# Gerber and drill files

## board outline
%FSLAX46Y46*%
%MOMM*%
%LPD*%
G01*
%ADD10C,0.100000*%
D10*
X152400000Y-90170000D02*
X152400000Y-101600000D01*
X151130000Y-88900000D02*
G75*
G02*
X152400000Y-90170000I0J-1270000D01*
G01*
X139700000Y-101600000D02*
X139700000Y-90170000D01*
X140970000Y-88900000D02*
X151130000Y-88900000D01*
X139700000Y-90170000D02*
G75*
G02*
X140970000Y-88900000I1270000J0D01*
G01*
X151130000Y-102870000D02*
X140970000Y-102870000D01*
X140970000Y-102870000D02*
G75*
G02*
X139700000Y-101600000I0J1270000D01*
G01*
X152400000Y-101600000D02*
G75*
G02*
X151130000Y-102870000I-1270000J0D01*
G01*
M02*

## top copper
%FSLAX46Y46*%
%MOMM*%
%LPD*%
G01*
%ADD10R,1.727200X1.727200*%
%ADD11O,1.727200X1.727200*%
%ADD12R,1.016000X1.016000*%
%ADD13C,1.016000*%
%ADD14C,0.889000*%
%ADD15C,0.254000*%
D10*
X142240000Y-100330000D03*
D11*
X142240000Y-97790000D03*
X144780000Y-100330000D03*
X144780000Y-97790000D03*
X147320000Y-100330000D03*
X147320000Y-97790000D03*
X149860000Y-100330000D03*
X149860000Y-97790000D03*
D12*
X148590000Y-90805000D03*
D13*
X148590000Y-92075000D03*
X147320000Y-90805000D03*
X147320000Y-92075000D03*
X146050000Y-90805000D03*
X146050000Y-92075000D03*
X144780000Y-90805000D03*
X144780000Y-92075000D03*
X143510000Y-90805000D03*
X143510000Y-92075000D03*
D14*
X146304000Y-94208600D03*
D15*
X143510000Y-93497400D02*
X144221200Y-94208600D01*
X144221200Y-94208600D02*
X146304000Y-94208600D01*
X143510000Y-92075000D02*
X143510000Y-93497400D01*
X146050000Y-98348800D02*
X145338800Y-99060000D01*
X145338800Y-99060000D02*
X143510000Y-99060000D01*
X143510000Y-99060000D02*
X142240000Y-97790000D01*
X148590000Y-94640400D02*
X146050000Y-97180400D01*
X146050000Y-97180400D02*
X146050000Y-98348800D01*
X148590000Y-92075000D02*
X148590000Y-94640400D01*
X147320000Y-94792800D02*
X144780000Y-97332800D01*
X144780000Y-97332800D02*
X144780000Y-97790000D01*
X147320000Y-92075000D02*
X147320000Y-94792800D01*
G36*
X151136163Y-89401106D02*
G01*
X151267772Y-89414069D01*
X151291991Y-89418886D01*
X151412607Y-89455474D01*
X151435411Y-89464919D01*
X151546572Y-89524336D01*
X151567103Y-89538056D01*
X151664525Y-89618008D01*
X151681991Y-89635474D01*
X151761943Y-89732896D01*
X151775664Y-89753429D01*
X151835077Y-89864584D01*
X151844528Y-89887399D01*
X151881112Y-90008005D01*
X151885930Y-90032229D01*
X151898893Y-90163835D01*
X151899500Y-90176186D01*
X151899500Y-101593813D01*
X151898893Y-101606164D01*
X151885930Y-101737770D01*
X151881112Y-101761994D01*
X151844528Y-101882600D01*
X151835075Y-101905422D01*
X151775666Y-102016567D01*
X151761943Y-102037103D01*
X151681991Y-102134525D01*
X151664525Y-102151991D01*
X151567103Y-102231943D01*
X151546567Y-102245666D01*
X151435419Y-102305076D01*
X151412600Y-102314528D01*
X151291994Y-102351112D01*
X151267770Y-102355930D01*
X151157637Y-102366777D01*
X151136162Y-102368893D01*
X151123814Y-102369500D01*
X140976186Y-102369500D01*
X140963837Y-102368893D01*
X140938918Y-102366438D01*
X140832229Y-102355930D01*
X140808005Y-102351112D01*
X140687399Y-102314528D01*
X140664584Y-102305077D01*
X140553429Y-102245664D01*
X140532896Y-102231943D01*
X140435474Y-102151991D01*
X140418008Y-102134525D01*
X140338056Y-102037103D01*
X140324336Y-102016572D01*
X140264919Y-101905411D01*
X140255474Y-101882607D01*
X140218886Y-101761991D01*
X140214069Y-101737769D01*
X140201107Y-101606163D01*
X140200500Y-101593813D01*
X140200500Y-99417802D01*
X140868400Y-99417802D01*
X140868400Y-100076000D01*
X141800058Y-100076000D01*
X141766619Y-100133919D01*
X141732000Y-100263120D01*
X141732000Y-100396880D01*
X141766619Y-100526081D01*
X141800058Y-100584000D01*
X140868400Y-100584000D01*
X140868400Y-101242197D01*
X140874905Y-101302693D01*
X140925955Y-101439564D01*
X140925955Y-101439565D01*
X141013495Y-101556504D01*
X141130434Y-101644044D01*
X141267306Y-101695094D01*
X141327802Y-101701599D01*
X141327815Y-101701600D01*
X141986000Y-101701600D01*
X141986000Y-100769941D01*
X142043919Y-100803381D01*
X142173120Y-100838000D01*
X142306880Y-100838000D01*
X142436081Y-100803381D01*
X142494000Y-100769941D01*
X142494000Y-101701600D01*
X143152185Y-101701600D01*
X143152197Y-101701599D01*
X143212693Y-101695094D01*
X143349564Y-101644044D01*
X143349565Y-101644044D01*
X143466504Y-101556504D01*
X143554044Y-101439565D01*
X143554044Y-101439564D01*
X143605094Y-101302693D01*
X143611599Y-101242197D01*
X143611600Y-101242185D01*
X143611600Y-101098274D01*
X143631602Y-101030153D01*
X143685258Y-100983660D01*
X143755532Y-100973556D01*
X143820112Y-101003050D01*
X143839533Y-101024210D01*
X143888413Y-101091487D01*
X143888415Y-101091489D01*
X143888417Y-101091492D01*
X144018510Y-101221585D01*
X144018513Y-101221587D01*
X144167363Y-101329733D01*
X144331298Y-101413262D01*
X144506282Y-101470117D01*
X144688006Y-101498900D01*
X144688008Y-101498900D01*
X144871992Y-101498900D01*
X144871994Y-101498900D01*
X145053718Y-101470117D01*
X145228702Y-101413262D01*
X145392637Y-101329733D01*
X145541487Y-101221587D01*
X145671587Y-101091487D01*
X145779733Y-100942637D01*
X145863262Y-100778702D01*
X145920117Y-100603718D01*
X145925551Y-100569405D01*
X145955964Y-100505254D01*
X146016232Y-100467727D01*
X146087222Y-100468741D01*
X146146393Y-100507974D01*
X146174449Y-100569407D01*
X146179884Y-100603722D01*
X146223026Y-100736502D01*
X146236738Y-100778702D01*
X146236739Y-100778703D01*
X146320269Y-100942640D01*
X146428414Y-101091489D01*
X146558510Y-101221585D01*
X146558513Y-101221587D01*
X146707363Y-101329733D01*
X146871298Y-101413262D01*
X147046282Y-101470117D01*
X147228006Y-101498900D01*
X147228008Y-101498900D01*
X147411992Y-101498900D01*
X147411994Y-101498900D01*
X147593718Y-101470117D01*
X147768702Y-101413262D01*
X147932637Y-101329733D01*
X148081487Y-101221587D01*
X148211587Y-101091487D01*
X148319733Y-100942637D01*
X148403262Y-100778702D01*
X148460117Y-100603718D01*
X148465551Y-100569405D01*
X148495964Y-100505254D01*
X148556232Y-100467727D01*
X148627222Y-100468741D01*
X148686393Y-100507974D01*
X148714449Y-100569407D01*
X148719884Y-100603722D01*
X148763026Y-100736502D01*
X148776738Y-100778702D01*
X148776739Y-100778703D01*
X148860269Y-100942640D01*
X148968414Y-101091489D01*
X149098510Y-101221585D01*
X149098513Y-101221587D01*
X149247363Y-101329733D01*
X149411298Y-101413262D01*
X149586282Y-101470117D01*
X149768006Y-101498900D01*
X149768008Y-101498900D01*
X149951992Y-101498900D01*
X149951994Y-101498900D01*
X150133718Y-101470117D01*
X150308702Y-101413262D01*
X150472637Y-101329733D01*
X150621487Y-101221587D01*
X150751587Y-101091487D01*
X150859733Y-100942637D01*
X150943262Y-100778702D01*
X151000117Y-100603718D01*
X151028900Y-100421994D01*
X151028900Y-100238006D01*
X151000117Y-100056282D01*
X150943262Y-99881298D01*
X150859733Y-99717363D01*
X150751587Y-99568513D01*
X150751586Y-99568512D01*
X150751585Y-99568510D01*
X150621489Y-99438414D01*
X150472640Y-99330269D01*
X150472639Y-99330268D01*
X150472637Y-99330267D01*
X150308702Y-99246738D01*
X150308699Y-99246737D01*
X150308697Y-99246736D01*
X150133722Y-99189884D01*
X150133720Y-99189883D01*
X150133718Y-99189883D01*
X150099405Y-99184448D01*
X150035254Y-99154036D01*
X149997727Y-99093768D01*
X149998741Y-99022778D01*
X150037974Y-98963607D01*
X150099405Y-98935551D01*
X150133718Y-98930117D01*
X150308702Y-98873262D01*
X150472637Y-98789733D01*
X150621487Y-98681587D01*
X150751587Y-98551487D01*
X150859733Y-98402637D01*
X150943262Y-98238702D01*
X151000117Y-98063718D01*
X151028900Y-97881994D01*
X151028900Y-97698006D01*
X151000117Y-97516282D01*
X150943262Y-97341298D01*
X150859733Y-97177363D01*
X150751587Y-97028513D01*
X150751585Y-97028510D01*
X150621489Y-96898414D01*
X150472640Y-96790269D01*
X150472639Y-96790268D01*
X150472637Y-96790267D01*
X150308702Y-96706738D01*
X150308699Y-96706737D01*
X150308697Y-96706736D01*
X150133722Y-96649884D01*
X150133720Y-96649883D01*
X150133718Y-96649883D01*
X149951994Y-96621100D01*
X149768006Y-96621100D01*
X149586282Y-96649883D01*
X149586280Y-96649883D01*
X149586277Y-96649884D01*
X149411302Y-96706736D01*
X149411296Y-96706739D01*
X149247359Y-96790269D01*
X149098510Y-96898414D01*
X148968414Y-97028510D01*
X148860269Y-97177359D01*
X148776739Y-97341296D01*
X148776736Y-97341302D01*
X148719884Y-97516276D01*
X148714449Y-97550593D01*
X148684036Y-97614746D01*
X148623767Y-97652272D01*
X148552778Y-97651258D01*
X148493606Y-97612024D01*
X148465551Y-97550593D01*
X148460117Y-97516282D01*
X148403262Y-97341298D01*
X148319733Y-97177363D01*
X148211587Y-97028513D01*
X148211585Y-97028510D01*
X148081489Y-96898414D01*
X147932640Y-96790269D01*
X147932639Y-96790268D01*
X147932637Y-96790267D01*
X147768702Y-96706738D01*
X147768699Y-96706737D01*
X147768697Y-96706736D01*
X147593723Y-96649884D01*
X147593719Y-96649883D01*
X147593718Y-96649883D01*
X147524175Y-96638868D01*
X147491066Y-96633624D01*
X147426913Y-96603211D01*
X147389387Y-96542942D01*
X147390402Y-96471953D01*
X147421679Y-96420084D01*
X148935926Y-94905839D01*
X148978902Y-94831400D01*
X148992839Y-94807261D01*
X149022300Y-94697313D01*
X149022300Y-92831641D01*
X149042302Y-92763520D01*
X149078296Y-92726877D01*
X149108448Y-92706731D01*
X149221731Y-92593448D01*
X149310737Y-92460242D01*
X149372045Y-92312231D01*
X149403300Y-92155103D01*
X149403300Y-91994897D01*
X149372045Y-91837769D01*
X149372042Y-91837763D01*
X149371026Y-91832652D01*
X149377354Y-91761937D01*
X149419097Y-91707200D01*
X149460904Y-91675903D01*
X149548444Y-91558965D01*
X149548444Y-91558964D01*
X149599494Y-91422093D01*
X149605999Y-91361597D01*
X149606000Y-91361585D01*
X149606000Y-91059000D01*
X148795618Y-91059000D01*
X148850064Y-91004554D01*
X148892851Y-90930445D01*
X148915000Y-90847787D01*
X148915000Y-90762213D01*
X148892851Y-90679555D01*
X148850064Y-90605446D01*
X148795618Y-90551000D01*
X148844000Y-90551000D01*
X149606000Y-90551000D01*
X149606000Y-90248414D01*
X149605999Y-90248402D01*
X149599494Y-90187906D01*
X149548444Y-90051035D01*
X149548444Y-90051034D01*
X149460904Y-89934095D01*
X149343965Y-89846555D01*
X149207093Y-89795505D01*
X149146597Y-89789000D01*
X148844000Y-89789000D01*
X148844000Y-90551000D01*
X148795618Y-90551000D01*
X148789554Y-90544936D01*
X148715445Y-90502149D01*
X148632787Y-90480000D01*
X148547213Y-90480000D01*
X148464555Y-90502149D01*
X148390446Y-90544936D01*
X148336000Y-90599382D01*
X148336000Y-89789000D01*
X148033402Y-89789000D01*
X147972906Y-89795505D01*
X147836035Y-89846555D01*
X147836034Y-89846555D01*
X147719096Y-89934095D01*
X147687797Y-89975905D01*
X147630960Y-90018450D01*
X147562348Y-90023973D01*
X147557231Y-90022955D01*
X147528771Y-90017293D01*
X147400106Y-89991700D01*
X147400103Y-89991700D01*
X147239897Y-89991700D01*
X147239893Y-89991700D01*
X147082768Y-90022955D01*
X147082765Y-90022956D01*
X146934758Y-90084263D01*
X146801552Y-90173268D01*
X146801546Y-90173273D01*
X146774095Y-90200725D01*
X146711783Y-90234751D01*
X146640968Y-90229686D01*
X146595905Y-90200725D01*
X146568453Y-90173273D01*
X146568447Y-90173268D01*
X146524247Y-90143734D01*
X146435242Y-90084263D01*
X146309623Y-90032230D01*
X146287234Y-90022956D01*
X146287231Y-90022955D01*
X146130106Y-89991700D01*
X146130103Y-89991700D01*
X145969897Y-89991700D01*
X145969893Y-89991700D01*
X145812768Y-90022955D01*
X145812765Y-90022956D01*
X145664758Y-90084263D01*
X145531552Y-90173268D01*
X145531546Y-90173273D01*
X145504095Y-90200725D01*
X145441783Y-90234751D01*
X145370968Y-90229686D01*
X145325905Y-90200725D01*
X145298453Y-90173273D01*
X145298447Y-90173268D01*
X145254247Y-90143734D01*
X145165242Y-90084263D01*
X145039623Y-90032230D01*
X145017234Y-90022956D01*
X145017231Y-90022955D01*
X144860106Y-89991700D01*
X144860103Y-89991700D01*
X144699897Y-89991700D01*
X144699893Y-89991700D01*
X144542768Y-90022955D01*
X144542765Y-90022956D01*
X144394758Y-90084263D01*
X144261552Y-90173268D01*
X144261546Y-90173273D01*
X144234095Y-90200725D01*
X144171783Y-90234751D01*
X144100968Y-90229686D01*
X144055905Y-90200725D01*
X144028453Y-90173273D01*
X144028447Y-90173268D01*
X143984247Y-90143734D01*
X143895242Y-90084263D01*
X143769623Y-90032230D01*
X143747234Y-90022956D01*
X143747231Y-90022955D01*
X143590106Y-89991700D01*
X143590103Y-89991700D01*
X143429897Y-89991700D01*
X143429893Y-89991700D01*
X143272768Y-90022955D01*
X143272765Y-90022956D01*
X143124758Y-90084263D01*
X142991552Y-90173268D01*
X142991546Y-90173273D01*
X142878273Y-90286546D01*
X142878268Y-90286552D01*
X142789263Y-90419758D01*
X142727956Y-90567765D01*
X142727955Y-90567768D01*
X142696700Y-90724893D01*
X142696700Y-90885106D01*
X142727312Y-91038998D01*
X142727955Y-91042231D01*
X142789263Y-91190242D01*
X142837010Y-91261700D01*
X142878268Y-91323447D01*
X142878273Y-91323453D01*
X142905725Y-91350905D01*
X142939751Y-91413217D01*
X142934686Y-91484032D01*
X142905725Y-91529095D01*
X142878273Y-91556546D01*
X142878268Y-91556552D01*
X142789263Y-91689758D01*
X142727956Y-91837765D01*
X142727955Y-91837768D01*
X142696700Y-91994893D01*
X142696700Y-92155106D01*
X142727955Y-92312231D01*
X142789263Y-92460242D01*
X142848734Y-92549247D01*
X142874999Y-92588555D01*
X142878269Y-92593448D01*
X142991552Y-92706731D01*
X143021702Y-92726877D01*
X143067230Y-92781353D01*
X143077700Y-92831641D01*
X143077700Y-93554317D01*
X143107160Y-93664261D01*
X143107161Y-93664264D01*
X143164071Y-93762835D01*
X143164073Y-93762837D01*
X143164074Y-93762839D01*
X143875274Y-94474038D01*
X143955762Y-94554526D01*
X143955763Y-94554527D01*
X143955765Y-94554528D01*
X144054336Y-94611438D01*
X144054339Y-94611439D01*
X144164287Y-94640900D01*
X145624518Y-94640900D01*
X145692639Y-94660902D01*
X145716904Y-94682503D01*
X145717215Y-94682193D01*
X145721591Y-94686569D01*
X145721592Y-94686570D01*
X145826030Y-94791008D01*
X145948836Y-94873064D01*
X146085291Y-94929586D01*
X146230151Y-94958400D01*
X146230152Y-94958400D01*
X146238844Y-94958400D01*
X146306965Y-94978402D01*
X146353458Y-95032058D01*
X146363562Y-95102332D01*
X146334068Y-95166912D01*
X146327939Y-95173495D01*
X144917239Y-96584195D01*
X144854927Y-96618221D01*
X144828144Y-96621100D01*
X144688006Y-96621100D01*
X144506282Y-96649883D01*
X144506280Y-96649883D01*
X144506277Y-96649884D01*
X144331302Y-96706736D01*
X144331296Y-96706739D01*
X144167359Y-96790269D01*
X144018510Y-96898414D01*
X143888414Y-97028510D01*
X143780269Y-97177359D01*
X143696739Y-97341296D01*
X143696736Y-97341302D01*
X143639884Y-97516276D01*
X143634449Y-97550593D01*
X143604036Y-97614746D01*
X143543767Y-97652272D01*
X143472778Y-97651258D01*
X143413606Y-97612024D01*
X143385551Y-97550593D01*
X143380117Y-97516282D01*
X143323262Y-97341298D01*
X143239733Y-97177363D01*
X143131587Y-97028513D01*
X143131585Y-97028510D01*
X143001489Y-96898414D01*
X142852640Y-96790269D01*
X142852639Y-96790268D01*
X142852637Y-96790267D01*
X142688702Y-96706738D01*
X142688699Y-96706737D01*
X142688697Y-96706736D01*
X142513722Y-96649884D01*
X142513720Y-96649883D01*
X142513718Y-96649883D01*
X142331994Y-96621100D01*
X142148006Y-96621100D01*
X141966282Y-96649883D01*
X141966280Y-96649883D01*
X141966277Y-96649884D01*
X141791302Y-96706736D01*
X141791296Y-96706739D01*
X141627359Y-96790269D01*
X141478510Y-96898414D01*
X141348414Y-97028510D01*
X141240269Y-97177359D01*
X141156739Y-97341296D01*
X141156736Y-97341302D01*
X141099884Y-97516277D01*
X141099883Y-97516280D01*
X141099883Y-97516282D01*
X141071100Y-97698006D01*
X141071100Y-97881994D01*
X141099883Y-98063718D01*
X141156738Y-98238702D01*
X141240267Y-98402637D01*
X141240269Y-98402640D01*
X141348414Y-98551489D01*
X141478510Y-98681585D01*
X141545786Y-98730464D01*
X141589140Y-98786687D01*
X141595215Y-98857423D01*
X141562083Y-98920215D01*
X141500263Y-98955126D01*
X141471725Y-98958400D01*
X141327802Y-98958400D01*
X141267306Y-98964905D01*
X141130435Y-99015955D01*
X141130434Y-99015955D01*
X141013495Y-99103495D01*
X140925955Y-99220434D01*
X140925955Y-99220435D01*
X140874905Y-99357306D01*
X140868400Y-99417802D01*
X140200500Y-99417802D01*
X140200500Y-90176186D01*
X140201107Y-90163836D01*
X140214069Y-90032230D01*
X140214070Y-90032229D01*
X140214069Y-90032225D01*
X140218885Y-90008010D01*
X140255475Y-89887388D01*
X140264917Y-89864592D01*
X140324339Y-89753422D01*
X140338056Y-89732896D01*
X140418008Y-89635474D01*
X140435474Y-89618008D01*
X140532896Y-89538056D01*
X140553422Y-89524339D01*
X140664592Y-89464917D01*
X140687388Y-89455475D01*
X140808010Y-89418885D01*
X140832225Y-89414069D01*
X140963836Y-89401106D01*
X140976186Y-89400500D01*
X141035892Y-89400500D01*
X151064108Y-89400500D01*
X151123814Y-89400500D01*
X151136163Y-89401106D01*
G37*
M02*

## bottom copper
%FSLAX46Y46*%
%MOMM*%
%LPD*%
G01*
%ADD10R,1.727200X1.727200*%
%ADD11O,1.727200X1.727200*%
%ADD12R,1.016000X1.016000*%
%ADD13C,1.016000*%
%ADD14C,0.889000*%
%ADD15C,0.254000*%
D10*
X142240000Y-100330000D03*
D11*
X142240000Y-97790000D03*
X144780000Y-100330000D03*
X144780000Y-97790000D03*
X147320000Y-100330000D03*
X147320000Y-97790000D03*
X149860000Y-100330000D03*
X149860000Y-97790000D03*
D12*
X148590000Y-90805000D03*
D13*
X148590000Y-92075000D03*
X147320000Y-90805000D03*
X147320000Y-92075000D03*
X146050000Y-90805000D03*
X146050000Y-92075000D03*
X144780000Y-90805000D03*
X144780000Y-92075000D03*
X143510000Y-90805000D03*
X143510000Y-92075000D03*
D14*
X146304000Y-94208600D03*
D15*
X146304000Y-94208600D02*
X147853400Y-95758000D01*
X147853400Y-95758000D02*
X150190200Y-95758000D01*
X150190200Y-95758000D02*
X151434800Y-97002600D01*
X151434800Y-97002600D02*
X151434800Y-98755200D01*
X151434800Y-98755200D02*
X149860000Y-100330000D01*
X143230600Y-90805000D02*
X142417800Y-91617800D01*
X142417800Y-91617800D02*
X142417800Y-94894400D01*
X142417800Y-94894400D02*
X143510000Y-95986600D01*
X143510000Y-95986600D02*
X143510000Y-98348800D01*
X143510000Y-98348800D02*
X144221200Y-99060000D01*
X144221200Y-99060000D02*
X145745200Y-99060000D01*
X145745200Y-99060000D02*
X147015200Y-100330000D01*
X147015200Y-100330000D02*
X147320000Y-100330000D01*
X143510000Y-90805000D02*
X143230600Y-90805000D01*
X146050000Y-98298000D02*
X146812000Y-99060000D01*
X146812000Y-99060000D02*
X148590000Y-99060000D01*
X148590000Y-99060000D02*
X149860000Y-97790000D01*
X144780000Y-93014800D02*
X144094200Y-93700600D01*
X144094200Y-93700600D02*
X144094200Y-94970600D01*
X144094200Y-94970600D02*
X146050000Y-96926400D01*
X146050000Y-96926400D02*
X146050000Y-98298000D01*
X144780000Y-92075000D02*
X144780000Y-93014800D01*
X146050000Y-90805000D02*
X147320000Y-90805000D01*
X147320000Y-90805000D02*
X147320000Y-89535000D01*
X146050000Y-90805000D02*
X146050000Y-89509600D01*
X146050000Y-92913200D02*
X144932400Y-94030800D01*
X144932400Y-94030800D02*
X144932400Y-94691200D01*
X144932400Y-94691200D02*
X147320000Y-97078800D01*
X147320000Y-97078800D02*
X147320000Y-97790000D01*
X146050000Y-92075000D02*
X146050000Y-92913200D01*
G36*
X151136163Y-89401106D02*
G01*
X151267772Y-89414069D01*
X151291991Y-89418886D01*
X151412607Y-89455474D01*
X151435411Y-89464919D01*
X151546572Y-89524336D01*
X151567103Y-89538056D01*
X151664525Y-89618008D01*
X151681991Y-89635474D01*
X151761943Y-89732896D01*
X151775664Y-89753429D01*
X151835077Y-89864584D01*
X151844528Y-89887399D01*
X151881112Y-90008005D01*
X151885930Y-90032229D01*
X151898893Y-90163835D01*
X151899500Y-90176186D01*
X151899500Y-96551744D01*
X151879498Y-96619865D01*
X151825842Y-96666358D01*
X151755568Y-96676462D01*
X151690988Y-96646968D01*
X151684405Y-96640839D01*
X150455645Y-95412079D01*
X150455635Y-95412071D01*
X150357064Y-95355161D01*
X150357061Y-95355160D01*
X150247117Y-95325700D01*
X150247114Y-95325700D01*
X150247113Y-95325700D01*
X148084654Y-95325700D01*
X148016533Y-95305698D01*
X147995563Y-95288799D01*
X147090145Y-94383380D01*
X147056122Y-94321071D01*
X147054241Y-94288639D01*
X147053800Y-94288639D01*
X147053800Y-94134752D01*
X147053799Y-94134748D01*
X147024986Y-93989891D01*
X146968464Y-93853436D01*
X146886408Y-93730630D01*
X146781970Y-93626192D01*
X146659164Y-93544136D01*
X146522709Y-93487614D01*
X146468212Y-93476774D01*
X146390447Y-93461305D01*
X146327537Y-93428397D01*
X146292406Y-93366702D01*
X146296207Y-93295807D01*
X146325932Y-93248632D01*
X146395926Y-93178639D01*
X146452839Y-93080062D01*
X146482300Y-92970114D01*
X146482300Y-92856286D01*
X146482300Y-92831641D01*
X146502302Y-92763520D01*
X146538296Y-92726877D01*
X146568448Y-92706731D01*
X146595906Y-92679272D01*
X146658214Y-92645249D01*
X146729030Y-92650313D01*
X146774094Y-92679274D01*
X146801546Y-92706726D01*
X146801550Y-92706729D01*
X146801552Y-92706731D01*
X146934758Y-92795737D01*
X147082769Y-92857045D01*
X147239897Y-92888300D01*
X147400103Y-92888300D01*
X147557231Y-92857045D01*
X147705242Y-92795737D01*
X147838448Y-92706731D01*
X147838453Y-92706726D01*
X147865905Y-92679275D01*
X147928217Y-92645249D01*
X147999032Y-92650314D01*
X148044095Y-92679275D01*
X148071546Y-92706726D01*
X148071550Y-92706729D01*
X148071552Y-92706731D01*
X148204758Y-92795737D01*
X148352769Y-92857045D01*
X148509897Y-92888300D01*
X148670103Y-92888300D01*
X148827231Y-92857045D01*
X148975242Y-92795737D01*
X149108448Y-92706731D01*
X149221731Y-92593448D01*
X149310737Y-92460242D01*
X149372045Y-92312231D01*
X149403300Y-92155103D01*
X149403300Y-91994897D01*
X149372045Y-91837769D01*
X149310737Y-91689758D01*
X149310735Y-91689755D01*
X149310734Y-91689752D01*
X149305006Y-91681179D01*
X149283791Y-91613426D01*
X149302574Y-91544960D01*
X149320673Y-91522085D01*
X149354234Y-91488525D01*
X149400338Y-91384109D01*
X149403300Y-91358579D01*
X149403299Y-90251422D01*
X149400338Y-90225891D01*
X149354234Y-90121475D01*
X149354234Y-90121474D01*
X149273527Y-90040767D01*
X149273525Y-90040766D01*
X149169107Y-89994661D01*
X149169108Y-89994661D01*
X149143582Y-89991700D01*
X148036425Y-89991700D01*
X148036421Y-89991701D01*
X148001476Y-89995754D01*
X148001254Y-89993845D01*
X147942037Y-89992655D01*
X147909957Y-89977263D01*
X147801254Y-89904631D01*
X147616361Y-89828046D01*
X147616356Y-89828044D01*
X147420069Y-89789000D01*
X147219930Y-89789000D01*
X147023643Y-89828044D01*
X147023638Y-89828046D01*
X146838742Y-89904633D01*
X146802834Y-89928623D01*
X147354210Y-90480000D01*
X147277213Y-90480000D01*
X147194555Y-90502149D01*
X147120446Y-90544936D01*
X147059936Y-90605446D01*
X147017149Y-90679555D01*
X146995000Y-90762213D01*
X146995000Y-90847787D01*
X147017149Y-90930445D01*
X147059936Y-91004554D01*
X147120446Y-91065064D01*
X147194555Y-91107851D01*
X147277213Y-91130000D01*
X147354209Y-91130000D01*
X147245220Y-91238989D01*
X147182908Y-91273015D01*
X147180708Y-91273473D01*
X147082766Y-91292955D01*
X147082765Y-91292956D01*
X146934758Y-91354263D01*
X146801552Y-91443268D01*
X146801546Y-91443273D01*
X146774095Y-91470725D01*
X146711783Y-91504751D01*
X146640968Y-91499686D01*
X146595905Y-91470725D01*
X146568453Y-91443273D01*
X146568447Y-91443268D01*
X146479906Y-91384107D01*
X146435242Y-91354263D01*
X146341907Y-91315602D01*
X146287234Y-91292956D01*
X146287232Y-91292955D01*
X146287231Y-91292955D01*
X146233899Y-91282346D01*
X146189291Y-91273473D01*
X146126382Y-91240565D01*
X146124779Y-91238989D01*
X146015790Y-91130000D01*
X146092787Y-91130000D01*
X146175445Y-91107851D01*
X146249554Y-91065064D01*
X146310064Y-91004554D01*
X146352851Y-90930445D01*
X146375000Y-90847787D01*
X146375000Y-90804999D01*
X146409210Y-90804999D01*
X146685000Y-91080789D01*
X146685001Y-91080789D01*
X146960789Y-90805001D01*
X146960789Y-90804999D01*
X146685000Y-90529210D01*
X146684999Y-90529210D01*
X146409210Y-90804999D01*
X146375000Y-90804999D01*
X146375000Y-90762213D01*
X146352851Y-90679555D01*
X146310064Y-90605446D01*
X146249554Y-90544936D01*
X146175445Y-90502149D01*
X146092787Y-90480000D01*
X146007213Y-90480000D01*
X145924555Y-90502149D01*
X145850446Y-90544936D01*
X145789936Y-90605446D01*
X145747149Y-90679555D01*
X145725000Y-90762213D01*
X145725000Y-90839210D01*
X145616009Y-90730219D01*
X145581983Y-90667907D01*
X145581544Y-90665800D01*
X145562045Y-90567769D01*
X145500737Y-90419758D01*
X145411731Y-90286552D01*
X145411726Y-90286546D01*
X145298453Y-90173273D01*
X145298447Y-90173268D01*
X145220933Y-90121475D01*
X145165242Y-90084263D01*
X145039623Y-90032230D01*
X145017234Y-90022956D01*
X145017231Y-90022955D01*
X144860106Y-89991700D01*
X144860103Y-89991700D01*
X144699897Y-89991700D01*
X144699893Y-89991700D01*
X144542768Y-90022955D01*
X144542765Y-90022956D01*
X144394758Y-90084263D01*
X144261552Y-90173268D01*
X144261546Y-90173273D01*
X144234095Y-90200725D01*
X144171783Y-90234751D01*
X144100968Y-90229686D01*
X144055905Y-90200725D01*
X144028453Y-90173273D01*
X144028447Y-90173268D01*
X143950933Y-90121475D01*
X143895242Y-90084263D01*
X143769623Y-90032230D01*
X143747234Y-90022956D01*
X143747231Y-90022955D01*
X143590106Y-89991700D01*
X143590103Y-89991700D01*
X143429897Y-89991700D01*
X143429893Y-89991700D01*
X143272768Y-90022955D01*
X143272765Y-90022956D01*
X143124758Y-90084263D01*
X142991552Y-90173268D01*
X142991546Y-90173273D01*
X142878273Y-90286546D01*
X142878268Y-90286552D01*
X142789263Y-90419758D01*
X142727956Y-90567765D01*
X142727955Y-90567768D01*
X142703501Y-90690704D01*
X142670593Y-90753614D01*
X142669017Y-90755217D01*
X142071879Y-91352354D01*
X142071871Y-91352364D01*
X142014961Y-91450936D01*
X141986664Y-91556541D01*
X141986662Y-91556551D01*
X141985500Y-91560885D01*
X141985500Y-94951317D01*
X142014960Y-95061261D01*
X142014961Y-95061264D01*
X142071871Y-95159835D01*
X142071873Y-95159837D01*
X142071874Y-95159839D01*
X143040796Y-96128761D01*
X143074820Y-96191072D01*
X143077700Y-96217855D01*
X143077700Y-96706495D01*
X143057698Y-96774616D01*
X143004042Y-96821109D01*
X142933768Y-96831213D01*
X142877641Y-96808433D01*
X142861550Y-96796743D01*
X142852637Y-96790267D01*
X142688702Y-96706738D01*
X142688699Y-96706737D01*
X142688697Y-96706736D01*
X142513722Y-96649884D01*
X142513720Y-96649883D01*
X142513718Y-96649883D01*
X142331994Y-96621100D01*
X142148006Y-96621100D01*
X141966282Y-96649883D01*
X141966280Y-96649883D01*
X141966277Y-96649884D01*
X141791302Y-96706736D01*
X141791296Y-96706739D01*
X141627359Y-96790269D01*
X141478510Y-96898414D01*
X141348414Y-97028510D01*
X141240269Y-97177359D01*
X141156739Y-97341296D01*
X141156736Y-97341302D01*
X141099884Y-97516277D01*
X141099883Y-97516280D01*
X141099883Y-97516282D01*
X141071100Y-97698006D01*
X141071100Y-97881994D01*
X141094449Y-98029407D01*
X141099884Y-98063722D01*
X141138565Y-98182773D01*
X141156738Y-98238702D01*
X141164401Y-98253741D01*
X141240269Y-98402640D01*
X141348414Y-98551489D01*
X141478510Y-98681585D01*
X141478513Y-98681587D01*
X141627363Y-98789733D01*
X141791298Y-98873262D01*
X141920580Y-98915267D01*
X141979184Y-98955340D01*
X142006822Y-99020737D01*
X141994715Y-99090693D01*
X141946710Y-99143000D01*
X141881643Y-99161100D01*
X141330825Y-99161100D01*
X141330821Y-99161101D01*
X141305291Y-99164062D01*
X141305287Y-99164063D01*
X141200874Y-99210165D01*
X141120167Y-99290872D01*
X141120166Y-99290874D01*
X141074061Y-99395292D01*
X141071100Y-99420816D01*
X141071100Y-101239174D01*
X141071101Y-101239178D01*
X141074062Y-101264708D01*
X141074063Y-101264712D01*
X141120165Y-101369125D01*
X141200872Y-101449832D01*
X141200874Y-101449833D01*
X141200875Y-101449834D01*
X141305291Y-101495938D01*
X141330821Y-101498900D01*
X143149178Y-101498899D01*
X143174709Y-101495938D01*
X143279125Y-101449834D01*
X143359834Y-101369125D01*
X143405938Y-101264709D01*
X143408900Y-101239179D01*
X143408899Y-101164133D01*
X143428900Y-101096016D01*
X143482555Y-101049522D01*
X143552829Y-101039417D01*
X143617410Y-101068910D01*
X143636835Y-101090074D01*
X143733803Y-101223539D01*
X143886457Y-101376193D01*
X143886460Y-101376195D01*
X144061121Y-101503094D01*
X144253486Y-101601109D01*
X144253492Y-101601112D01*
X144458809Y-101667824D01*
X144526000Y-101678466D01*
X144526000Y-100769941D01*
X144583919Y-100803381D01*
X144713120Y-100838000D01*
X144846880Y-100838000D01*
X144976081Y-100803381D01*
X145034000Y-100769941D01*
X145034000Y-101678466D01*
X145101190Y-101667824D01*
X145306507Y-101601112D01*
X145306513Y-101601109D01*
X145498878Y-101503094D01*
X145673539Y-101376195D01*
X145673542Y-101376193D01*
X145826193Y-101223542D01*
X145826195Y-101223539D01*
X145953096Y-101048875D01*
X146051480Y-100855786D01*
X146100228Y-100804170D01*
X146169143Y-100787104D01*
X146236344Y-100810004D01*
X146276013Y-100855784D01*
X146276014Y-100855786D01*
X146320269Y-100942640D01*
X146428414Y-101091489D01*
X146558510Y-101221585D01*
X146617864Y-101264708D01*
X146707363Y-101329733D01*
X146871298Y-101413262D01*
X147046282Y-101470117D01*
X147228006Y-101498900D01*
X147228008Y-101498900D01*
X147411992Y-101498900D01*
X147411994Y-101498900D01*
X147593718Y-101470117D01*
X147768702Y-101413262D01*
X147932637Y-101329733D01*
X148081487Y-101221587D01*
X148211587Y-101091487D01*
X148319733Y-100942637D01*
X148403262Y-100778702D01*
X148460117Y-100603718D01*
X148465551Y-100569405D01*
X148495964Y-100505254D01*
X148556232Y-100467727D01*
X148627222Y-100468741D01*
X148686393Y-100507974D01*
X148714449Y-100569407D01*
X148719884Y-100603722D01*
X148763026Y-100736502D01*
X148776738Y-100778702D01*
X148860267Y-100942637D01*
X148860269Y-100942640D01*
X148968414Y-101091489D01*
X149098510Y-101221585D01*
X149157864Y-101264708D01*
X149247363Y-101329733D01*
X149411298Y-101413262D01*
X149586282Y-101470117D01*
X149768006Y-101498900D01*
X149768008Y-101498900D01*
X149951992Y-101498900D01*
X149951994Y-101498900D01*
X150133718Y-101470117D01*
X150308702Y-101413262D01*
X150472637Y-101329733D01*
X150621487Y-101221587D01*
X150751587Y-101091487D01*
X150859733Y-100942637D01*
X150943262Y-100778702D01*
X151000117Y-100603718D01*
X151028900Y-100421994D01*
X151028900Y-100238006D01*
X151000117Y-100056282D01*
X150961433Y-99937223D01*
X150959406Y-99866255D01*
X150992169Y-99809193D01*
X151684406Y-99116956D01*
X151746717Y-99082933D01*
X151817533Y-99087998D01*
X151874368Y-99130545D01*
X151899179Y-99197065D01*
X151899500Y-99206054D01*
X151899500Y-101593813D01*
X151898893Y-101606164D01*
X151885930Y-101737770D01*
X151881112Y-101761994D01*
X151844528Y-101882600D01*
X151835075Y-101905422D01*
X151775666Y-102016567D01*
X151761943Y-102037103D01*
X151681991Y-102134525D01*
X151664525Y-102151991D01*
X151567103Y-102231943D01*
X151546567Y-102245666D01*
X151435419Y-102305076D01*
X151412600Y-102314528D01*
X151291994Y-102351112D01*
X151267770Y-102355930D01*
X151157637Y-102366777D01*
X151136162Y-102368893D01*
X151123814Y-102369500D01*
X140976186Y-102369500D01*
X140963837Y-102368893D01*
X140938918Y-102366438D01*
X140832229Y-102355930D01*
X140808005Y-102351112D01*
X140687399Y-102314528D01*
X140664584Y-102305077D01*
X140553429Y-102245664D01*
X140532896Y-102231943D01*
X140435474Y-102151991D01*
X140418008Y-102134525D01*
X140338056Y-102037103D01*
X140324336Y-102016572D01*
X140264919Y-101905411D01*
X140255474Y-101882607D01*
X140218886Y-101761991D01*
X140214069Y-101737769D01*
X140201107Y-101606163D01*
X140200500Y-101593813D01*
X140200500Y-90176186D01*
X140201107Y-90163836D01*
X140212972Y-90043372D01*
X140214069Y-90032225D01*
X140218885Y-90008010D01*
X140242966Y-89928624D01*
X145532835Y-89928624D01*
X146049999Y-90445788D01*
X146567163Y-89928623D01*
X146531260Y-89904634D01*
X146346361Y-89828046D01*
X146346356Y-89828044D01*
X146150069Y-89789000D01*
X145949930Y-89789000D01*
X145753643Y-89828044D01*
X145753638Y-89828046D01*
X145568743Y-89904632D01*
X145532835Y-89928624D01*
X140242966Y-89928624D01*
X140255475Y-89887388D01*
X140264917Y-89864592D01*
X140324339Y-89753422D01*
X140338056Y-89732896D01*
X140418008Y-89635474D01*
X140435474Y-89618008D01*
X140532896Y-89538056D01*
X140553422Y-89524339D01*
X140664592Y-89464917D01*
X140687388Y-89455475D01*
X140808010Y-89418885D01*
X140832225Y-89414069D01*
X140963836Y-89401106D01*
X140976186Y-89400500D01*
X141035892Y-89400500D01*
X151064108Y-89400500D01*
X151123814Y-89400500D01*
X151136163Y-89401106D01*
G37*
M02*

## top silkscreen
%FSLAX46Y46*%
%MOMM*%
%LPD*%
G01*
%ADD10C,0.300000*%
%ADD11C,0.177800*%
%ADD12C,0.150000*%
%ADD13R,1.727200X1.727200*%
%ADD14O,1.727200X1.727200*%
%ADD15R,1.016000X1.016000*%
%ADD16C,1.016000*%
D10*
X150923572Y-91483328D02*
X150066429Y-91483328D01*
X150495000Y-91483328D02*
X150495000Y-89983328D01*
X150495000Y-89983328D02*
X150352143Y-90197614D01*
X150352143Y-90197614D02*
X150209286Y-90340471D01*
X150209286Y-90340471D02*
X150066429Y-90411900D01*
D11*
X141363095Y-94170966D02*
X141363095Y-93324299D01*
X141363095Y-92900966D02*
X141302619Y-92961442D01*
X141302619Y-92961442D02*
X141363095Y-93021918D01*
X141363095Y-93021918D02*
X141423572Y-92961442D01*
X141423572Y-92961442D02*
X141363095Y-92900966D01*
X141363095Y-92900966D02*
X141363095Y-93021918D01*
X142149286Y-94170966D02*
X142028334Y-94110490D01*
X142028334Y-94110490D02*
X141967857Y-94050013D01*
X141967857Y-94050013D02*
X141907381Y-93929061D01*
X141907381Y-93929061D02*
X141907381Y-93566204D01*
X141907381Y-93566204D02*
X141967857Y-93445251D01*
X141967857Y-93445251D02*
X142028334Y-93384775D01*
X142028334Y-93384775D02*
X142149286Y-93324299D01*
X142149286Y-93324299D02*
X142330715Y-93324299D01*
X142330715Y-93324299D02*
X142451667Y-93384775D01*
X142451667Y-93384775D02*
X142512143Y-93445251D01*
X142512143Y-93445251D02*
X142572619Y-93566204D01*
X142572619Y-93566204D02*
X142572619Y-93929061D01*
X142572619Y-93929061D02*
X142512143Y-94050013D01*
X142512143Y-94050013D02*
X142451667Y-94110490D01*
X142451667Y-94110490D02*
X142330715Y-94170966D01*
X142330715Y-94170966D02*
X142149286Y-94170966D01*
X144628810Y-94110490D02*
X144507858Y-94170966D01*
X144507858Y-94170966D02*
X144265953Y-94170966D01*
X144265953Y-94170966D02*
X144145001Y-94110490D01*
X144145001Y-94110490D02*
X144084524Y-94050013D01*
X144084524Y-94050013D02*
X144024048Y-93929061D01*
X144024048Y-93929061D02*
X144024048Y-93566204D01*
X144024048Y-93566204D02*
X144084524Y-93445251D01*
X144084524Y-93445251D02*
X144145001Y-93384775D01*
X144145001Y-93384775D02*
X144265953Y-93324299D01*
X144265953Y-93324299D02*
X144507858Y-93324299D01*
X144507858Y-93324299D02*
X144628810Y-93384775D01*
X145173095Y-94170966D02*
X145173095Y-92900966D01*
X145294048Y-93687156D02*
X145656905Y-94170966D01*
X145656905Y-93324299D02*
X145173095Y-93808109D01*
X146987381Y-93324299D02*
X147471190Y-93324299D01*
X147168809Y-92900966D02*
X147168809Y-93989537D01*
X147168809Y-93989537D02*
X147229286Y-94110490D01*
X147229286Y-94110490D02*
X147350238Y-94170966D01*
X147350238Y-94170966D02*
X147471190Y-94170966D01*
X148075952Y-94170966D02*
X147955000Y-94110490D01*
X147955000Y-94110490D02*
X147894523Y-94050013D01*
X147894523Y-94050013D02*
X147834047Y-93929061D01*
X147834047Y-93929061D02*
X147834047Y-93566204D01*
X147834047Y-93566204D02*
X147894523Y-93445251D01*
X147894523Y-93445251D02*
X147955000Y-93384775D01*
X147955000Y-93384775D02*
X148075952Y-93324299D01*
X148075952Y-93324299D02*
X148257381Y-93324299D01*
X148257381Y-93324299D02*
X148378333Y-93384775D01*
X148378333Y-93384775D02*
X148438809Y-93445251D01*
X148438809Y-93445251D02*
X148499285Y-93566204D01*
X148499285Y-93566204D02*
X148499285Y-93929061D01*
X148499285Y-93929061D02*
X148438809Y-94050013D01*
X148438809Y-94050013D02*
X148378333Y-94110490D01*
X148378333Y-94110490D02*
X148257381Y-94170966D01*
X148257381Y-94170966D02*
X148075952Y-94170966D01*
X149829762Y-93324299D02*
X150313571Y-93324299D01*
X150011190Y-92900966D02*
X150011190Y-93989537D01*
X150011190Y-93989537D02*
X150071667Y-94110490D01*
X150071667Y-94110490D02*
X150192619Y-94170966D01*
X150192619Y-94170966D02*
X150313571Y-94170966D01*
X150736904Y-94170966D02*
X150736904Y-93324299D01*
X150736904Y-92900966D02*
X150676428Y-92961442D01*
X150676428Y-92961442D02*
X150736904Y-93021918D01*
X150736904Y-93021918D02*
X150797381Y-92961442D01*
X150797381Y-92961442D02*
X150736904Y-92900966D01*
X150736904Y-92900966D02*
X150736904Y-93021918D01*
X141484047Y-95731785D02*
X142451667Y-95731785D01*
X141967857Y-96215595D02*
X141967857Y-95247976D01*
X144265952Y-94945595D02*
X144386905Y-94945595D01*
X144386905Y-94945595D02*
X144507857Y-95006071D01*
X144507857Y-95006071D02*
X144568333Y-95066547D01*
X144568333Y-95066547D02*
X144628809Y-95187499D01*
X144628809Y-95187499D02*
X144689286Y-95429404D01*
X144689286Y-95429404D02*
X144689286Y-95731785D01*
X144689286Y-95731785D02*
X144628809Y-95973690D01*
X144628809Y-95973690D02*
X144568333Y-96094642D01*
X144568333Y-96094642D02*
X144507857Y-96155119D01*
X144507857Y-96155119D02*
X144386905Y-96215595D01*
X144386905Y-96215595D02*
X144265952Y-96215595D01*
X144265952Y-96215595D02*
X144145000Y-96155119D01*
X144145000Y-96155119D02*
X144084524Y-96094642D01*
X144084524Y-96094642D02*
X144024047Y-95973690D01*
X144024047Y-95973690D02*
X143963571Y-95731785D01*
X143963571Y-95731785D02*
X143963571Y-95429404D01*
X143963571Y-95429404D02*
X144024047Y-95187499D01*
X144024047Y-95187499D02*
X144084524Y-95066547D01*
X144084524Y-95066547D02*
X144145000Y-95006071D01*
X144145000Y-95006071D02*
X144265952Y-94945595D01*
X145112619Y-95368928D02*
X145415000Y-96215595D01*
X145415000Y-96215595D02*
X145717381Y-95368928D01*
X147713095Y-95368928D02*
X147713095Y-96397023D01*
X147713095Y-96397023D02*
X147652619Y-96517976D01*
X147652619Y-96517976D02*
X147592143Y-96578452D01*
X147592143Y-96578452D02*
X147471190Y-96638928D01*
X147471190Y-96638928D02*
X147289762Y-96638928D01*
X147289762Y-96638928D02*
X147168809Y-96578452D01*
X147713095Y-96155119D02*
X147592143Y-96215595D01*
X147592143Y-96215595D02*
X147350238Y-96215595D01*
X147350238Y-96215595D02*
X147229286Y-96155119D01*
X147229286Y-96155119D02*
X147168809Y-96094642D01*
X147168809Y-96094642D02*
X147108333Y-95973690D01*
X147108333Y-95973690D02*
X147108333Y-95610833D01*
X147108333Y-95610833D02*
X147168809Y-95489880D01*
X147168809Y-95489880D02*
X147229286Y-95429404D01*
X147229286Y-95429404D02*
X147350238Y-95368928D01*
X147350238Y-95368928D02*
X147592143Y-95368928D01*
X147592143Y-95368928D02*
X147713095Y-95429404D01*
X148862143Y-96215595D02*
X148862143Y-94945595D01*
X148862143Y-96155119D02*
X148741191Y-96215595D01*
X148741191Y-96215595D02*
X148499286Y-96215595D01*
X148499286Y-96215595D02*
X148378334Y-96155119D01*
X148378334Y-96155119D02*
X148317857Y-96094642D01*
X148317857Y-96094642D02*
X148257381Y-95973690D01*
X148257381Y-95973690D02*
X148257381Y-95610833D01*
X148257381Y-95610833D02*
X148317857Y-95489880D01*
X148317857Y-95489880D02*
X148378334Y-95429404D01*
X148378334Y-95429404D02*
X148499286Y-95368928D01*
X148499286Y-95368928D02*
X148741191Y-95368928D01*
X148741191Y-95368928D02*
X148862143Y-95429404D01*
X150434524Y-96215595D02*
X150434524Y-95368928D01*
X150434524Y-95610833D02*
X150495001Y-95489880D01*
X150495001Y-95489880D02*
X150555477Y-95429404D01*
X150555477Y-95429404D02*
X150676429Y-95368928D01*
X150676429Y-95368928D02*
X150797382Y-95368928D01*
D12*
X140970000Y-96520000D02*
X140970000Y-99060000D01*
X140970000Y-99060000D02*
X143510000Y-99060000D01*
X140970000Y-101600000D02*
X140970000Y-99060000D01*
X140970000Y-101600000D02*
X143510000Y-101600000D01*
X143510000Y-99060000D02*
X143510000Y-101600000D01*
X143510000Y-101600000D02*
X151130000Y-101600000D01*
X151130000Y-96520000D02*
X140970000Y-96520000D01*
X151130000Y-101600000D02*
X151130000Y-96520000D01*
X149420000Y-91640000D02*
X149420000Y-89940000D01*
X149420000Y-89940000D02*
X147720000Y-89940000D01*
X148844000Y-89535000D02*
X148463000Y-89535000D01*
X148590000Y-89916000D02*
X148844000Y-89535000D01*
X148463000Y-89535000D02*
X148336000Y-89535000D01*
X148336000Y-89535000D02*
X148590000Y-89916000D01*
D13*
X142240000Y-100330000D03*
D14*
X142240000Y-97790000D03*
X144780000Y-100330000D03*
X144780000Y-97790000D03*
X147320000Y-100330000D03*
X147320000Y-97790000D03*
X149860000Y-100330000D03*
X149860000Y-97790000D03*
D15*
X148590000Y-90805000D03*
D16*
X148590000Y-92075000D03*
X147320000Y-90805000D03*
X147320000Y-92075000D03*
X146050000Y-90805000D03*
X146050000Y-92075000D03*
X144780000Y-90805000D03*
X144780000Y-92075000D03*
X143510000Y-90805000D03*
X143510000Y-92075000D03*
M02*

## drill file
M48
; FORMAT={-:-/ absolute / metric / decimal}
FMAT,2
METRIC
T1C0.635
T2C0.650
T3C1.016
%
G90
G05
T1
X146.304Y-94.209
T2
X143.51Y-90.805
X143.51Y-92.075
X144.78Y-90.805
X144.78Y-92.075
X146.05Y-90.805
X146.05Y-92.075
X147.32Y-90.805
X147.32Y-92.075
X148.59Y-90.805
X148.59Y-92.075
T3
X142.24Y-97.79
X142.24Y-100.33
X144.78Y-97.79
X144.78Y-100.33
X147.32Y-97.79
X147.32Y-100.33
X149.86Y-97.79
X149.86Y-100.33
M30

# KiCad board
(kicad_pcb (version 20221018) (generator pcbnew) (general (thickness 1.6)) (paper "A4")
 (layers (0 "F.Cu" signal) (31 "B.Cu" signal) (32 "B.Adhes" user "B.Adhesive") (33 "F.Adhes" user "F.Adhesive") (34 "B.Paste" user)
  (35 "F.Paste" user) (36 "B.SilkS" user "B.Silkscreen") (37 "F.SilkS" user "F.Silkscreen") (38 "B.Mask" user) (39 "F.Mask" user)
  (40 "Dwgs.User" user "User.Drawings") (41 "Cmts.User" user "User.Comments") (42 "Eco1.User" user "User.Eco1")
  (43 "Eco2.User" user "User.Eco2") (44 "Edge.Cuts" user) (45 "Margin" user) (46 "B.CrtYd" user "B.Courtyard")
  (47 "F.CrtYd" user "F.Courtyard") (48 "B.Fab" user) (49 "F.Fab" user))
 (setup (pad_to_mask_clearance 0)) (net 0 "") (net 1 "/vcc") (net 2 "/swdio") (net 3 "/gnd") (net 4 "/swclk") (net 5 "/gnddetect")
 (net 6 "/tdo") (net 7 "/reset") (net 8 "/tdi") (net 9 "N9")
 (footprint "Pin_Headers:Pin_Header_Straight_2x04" (layer "F.Cu") (at 146.05 99.06)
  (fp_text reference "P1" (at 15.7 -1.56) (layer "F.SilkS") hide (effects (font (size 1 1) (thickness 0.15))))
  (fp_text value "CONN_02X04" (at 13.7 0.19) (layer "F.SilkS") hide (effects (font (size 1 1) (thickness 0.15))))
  (fp_line (start -5.08 -2.54) (end -5.08 0) (stroke (width 0.15) (type solid)) (layer "F.SilkS"))
  (fp_line (start -5.08 0) (end -2.54 0) (stroke (width 0.15) (type solid)) (layer "F.SilkS"))
  (fp_line (start -5.08 2.54) (end -5.08 0) (stroke (width 0.15) (type solid)) (layer "F.SilkS"))
  (fp_line (start -5.08 2.54) (end -2.54 2.54) (stroke (width 0.15) (type solid)) (layer "F.SilkS"))
  (fp_line (start -2.54 0) (end -2.54 2.54) (stroke (width 0.15) (type solid)) (layer "F.SilkS"))
  (fp_line (start -2.54 2.54) (end 5.08 2.54) (stroke (width 0.15) (type solid)) (layer "F.SilkS"))
  (fp_line (start 5.08 -2.54) (end -5.08 -2.54) (stroke (width 0.15) (type solid)) (layer "F.SilkS"))
  (fp_line (start 5.08 2.54) (end 5.08 -2.54) (stroke (width 0.15) (type solid)) (layer "F.SilkS"))
  (pad "1" thru_hole rect (at -3.81 1.27) (size 1.7272 1.7272) (drill 1.016) (layers "*.Cu" "*.Mask" "F.SilkS") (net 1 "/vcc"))
  (pad "2" thru_hole oval (at -3.81 -1.27) (size 1.7272 1.7272) (drill 1.016) (layers "*.Cu" "*.Mask" "F.SilkS") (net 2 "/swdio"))
  (pad "3" thru_hole oval (at -1.27 1.27) (size 1.7272 1.7272) (drill 1.016) (layers "*.Cu" "*.Mask" "F.SilkS") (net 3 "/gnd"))
  (pad "4" thru_hole oval (at -1.27 -1.27) (size 1.7272 1.7272) (drill 1.016) (layers "*.Cu" "*.Mask" "F.SilkS") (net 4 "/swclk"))
  (pad "5" thru_hole oval (at 1.27 1.27) (size 1.7272 1.7272) (drill 1.016) (layers "*.Cu" "*.Mask" "F.SilkS") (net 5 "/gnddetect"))
  (pad "6" thru_hole oval (at 1.27 -1.27) (size 1.7272 1.7272) (drill 1.016) (layers "*.Cu" "*.Mask" "F.SilkS") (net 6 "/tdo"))
  (pad "7" thru_hole oval (at 3.81 1.27) (size 1.7272 1.7272) (drill 1.016) (layers "*.Cu" "*.Mask" "F.SilkS") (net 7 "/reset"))
  (pad "8" thru_hole oval (at 3.81 -1.27) (size 1.7272 1.7272) (drill 1.016) (layers "*.Cu" "*.Mask" "F.SilkS") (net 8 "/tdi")))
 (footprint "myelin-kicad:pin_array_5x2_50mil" (layer "F.Cu") (at 147.32 91.44 180)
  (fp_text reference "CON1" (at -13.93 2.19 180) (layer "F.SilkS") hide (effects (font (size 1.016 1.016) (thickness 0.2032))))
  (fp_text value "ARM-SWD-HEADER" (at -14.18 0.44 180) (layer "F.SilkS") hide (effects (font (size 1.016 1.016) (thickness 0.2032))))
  (fp_line (start -2.1 -0.2) (end -2.1 1.5) (stroke (width 0.15) (type solid)) (layer "F.SilkS"))
  (fp_line (start -2.1 1.5) (end -0.4 1.5) (stroke (width 0.15) (type solid)) (layer "F.SilkS"))
  (fp_line (start -1.524 1.905) (end -1.143 1.905) (stroke (width 0.15) (type solid)) (layer "F.SilkS"))
  (fp_line (start -1.27 1.524) (end -1.524 1.905) (stroke (width 0.15) (type solid)) (layer "F.SilkS"))
  (fp_line (start -1.143 1.905) (end -1.016 1.905) (stroke (width 0.15) (type solid)) (layer "F.SilkS"))
  (fp_line (start -1.016 1.905) (end -1.27 1.524) (stroke (width 0.15) (type solid)) (layer "F.SilkS"))
  (pad "1" thru_hole rect (at -1.27 0.635 180) (size 1.016 1.016) (drill 0.65) (layers "*.Cu" "*.Mask" "F.SilkS") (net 1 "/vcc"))
  (pad "2" thru_hole circle (at -1.27 -0.635 180) (size 1.016 1.016) (drill 0.65) (layers "*.Cu" "*.Mask" "F.SilkS") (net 2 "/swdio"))
  (pad "3" thru_hole circle (at 0 0.635 180) (size 1.016 1.016) (drill 0.65) (layers "*.Cu" "*.Mask" "F.SilkS") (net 3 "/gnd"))
  (pad "4" thru_hole circle (at 0 -0.635 180) (size 1.016 1.016) (drill 0.65) (layers "*.Cu" "*.Mask" "F.SilkS") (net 4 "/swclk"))
  (pad "5" thru_hole circle (at 1.27 0.635 180) (size 1.016 1.016) (drill 0.65) (layers "*.Cu" "*.Mask" "F.SilkS") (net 3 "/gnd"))
  (pad "6" thru_hole circle (at 1.27 -0.635 180) (size 1.016 1.016) (drill 0.65) (layers "*.Cu" "*.Mask" "F.SilkS") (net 6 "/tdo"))
  (pad "7" thru_hole circle (at 2.54 0.635 180) (size 1.016 1.016) (drill 0.65) (layers "*.Cu" "*.Mask" "F.SilkS") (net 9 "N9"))
  (pad "8" thru_hole circle (at 2.54 -0.635 180) (size 1.016 1.016) (drill 0.65) (layers "*.Cu" "*.Mask" "F.SilkS") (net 8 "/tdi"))
  (pad "9" thru_hole circle (at 3.81 0.635 180) (size 1.016 1.016) (drill 0.65) (layers "*.Cu" "*.Mask" "F.SilkS") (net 5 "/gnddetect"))
  (pad "10" thru_hole circle (at 3.81 -0.635 180) (size 1.016 1.016) (drill 0.65) (layers "*.Cu" "*.Mask" "F.SilkS") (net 7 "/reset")))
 (gr_line (start 152.4 90.17) (end 152.4 101.6) (stroke (width 0.1) (type solid)) (layer "Edge.Cuts"))
 (gr_arc (start 151.13 88.9) (mid 152.028026 89.271974) (end 152.4 90.17) (stroke (width 0.1) (type solid)) (layer "Edge.Cuts"))
 (gr_line (start 139.7 101.6) (end 139.7 90.17) (stroke (width 0.1) (type solid)) (layer "Edge.Cuts"))
 (gr_line (start 140.97 88.9) (end 151.13 88.9) (stroke (width 0.1) (type solid)) (layer "Edge.Cuts"))
 (gr_arc (start 139.7 90.17) (mid 140.071974 89.271974) (end 140.97 88.9) (stroke (width 0.1) (type solid)) (layer "Edge.Cuts"))
 (gr_line (start 151.13 102.87) (end 140.97 102.87) (stroke (width 0.1) (type solid)) (layer "Edge.Cuts"))
 (gr_arc (start 140.97 102.87) (mid 140.071974 102.498026) (end 139.7 101.6) (stroke (width 0.1) (type solid)) (layer "Edge.Cuts"))
 (gr_arc (start 152.4 101.6) (mid 152.028026 102.498026) (end 151.13 102.87) (stroke (width 0.1) (type solid)) (layer "Edge.Cuts"))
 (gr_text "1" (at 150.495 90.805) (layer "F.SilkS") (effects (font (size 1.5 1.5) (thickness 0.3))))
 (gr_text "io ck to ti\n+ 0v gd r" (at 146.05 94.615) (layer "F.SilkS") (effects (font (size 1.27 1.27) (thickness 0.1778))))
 (segment (start 143.51 93.4974) (end 144.2212 94.2086) (width 0.254) (layer "F.Cu") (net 7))
 (segment (start 144.2212 94.2086) (end 146.304 94.2086) (width 0.254) (layer "F.Cu") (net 7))
 (segment (start 143.51 92.075) (end 143.51 93.4974) (width 0.254) (layer "F.Cu") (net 7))
 (via (at 146.304 94.2086) (size 0.889) (drill 0.635) (layers "F.Cu" "B.Cu") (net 7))
 (segment (start 146.304 94.2086) (end 147.8534 95.758) (width 0.254) (layer "B.Cu") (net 7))
 (segment (start 147.8534 95.758) (end 150.1902 95.758) (width 0.254) (layer "B.Cu") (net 7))
 (segment (start 150.1902 95.758) (end 151.4348 97.0026) (width 0.254) (layer "B.Cu") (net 7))
 (segment (start 151.4348 97.0026) (end 151.4348 98.7552) (width 0.254) (layer "B.Cu") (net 7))
 (segment (start 151.4348 98.7552) (end 149.86 100.33) (width 0.254) (layer "B.Cu") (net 7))
 (segment (start 143.2306 90.805) (end 142.4178 91.6178) (width 0.254) (layer "B.Cu") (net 5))
 (segment (start 142.4178 91.6178) (end 142.4178 94.8944) (width 0.254) (layer "B.Cu") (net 5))
 (segment (start 142.4178 94.8944) (end 143.51 95.9866) (width 0.254) (layer "B.Cu") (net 5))
 (segment (start 143.51 95.9866) (end 143.51 98.3488) (width 0.254) (layer "B.Cu") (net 5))
 (segment (start 143.51 98.3488) (end 144.2212 99.06) (width 0.254) (layer "B.Cu") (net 5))
 (segment (start 144.2212 99.06) (end 145.7452 99.06) (width 0.254) (layer "B.Cu") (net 5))
 (segment (start 145.7452 99.06) (end 147.0152 100.33) (width 0.254) (layer "B.Cu") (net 5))
 (segment (start 147.0152 100.33) (end 147.32 100.33) (width 0.254) (layer "B.Cu") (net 5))
 (segment (start 143.51 90.805) (end 143.2306 90.805) (width 0.254) (layer "B.Cu") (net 5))
 (segment (start 146.05 98.298) (end 146.812 99.06) (width 0.254) (layer "B.Cu") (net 8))
 (segment (start 146.812 99.06) (end 148.59 99.06) (width 0.254) (layer "B.Cu") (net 8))
 (segment (start 148.59 99.06) (end 149.86 97.79) (width 0.254) (layer "B.Cu") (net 8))
 (segment (start 144.78 93.0148) (end 144.0942 93.7006) (width 0.254) (layer "B.Cu") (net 8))
 (segment (start 144.0942 93.7006) (end 144.0942 94.9706) (width 0.254) (layer "B.Cu") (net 8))
 (segment (start 144.0942 94.9706) (end 146.05 96.9264) (width 0.254) (layer "B.Cu") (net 8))
 (segment (start 146.05 96.9264) (end 146.05 98.298) (width 0.254) (layer "B.Cu") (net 8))
 (segment (start 144.78 92.075) (end 144.78 93.0148) (width 0.254) (layer "B.Cu") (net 8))
 (segment (start 146.05 98.3488) (end 145.3388 99.06) (width 0.254) (layer "F.Cu") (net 2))
 (segment (start 145.3388 99.06) (end 143.51 99.06) (width 0.254) (layer "F.Cu") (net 2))
 (segment (start 143.51 99.06) (end 142.24 97.79) (width 0.254) (layer "F.Cu") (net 2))
 (segment (start 148.59 94.6404) (end 146.05 97.1804) (width 0.254) (layer "F.Cu") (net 2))
 (segment (start 146.05 97.1804) (end 146.05 98.3488) (width 0.254) (layer "F.Cu") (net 2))
 (segment (start 148.59 92.075) (end 148.59 94.6404) (width 0.254) (layer "F.Cu") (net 2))
 (segment (start 146.05 90.805) (end 147.32 90.805) (width 0.254) (layer "B.Cu") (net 3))
 (segment (start 147.32 90.805) (end 147.32 89.535) (width 0.254) (layer "B.Cu") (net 3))
 (segment (start 146.05 90.805) (end 146.05 89.5096) (width 0.254) (layer "B.Cu") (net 3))
 (segment (start 147.32 94.7928) (end 144.78 97.3328) (width 0.254) (layer "F.Cu") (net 4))
 (segment (start 144.78 97.3328) (end 144.78 97.79) (width 0.254) (layer "F.Cu") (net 4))
 (segment (start 147.32 92.075) (end 147.32 94.7928) (width 0.254) (layer "F.Cu") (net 4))
 (segment (start 146.05 92.9132) (end 144.9324 94.0308) (width 0.254) (layer "B.Cu") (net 6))
 (segment (start 144.9324 94.0308) (end 144.9324 94.6912) (width 0.254) (layer "B.Cu") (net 6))
 (segment (start 144.9324 94.6912) (end 147.32 97.0788) (width 0.254) (layer "B.Cu") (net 6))
 (segment (start 147.32 97.0788) (end 147.32 97.79) (width 0.254) (layer "B.Cu") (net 6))
 (segment (start 146.05 92.075) (end 146.05 92.9132) (width 0.254) (layer "B.Cu") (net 6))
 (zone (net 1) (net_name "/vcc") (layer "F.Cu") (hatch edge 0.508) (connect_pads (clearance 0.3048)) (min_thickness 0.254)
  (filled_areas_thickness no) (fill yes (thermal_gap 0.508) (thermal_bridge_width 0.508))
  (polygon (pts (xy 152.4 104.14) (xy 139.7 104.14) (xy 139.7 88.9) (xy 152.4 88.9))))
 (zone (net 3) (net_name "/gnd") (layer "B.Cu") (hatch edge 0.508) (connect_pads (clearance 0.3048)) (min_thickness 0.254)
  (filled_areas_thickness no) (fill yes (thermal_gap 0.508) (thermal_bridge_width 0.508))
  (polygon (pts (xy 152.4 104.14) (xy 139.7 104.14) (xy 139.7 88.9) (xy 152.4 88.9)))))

